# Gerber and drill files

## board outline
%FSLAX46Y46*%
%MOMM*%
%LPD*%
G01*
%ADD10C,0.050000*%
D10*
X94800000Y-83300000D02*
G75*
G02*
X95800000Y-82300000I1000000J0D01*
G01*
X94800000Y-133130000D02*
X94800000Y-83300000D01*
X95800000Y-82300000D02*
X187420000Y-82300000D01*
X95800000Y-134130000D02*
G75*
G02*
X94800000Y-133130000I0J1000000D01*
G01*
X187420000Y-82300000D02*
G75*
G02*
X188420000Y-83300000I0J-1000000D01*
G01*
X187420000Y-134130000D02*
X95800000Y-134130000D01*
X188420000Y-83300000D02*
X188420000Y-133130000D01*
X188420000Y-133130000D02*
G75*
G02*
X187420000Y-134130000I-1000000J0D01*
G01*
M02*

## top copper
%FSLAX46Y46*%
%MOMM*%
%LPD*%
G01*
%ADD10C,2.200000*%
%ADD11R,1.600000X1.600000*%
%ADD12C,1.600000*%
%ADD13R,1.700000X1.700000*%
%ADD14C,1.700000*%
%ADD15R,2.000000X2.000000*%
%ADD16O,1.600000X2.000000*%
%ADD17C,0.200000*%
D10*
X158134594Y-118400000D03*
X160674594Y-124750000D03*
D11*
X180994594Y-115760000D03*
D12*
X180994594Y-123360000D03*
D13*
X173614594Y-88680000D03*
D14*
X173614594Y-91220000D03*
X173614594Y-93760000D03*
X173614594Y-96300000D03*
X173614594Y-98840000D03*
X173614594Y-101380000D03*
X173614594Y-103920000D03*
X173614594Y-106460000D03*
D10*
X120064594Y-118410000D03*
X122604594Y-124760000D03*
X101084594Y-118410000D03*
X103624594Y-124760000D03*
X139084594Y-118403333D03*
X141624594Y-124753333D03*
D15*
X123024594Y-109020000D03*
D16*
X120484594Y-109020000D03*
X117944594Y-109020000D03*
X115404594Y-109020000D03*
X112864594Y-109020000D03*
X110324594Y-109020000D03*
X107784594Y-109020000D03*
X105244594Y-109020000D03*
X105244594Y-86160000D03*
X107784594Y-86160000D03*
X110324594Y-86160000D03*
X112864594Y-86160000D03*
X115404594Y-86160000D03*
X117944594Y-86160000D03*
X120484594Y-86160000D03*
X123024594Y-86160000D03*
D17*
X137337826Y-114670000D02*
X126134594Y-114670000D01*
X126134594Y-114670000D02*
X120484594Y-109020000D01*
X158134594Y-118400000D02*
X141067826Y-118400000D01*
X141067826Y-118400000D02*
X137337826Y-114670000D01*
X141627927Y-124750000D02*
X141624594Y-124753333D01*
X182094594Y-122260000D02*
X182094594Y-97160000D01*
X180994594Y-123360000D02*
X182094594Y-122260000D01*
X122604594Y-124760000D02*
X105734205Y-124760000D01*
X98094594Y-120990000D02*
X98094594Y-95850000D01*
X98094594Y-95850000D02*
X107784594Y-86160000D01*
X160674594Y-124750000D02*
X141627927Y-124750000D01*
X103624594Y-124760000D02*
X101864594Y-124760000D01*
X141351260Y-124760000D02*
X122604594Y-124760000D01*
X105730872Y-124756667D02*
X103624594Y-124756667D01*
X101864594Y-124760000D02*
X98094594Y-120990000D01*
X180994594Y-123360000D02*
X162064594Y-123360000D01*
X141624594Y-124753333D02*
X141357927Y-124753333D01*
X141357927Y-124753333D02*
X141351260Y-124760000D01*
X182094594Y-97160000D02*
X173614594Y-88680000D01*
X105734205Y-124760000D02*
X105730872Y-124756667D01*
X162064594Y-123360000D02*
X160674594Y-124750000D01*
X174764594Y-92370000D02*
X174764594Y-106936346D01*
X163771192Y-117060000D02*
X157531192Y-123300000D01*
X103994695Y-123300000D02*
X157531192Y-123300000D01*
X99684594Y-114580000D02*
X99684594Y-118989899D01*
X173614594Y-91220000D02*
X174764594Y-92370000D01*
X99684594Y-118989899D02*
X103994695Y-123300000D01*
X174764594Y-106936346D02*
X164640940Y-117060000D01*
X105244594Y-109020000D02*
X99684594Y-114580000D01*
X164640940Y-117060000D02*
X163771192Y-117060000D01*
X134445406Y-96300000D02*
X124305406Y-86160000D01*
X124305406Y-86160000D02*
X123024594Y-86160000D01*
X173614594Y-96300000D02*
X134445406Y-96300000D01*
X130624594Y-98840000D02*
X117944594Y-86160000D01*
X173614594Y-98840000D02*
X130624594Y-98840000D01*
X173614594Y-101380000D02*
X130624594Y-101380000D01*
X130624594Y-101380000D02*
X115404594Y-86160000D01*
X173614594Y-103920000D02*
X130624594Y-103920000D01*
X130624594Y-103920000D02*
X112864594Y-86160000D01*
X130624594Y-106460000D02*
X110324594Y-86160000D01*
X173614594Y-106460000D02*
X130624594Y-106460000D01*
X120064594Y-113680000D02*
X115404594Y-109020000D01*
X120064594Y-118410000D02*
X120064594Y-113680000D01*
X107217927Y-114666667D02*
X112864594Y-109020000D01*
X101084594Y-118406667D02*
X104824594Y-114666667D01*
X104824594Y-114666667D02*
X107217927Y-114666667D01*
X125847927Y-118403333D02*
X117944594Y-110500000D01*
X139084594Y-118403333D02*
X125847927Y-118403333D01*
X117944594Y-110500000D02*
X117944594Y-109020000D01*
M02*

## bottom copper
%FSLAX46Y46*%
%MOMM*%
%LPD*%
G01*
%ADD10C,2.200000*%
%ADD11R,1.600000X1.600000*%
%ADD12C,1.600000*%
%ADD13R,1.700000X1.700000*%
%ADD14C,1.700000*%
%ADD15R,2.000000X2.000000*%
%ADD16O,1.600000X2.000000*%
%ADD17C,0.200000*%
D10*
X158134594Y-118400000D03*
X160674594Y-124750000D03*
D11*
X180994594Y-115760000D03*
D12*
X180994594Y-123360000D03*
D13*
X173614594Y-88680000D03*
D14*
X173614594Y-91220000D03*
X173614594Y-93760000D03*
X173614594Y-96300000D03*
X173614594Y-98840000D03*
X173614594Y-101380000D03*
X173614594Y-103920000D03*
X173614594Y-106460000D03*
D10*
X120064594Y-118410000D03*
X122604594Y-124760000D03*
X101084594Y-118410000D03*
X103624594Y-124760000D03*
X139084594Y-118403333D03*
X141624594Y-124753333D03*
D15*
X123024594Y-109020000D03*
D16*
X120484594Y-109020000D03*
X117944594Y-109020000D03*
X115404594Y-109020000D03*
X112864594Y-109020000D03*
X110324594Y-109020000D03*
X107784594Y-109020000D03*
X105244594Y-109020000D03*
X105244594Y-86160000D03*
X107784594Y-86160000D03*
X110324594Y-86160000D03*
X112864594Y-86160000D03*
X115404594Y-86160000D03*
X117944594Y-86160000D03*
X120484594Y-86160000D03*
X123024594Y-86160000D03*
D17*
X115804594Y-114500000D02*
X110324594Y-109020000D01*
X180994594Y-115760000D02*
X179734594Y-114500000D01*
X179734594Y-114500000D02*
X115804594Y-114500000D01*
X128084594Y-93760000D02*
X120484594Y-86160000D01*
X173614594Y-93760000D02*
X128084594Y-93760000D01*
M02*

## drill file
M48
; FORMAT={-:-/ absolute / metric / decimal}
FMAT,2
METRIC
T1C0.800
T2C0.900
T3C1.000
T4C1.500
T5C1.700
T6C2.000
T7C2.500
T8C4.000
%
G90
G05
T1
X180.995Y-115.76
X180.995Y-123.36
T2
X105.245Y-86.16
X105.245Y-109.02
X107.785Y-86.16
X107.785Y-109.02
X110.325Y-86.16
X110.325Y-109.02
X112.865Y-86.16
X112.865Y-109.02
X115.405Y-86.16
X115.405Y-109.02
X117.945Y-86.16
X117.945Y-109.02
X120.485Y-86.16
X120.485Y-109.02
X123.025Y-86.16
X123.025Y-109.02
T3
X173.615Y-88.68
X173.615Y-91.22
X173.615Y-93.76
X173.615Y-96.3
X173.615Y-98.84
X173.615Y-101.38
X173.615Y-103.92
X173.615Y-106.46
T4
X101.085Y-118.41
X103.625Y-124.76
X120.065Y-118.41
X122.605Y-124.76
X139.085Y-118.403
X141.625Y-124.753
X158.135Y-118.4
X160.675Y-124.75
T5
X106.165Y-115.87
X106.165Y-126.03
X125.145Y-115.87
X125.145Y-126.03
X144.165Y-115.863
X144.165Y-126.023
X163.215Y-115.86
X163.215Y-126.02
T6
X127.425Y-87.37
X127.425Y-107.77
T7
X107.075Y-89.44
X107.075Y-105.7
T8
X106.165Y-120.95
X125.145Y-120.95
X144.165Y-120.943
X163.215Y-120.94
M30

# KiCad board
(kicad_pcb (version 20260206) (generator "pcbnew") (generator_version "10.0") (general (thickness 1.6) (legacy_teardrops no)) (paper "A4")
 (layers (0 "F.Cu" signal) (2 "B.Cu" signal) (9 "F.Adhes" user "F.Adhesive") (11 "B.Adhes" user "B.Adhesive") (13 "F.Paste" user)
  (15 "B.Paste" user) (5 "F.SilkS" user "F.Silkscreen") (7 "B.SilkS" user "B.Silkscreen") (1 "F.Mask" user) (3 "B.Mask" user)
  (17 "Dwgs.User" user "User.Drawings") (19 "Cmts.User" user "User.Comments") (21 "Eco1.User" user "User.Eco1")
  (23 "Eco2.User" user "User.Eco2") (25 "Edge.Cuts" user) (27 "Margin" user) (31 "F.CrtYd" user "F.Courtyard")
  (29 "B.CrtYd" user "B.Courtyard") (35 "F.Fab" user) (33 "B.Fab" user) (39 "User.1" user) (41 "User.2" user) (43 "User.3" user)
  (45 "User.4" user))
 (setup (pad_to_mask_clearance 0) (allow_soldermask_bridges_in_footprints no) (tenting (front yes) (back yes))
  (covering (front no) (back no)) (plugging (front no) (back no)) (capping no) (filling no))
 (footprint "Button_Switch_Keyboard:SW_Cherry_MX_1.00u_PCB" (layer "F.Cu") (at 158.134594 118.4 90)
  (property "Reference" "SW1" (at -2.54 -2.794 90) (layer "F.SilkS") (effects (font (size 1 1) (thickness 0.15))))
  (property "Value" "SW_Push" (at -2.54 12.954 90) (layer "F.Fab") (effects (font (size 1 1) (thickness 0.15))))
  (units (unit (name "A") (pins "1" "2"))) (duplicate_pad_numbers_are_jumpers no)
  (pad "" np_thru_hole circle (at -7.62 5.08 90) (size 1.7 1.7) (drill 1.7) (layers "*.Cu" "*.Mask"))
  (pad "" np_thru_hole circle (at -2.54 5.08 90) (size 4 4) (drill 4) (layers "*.Cu" "*.Mask"))
  (pad "" np_thru_hole circle (at 2.54 5.08 90) (size 1.7 1.7) (drill 1.7) (layers "*.Cu" "*.Mask"))
  (pad "1" thru_hole circle (at 0 0 90) (size 2.2 2.2) (drill 1.5) (layers "*.Cu" "*.Mask") (remove_unused_layers no) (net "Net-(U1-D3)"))
  (pad "2" thru_hole circle (at -6.35 2.54 90) (size 2.2 2.2) (drill 1.5) (layers "*.Cu" "*.Mask") (remove_unused_layers no) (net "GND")))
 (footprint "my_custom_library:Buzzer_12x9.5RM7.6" (layer "F.Cu") (at 180.994594 119.56 -90)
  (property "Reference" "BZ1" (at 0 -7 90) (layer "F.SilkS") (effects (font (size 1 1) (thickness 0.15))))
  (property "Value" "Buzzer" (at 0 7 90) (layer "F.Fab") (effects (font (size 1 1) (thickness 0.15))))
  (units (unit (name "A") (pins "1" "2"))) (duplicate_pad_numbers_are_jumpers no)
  (pad "1" thru_hole rect (at -3.8 0 270) (size 1.6 1.6) (drill 0.8) (layers "*.Cu" "*.Mask") (remove_unused_layers no) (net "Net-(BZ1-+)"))
  (pad "2" thru_hole circle (at 3.8 0 270) (size 1.6 1.6) (drill 0.8) (layers "*.Cu" "*.Mask") (remove_unused_layers no) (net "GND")))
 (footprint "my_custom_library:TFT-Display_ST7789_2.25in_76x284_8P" (layer "F.Cu") (at 173.614594 88.68 -90)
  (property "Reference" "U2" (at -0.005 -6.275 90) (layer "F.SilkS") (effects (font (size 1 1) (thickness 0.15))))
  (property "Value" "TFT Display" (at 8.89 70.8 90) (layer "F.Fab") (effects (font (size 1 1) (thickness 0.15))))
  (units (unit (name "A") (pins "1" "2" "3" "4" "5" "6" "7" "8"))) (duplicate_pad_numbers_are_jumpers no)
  (pad "" np_thru_hole circle (at 0.76 66.54 270) (size 2.5 2.5) (drill 2.5) (layers "*.Cu" "*.Mask"))
  (pad "" np_thru_hole circle (at 17.02 66.54 270) (size 2.5 2.5) (drill 2.5) (layers "*.Cu" "*.Mask"))
  (pad "1" thru_hole rect (at 0 0 270) (size 1.7 1.7) (drill 1) (layers "*.Cu" "*.Mask") (remove_unused_layers no) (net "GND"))
  (pad "2" thru_hole circle (at 2.54 0 270) (size 1.7 1.7) (drill 1) (layers "*.Cu" "*.Mask") (remove_unused_layers no) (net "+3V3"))
  (pad "3" thru_hole circle (at 5.08 0 270) (size 1.7 1.7) (drill 1) (layers "*.Cu" "*.Mask") (remove_unused_layers no) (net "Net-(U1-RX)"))
  (pad "4" thru_hole circle (at 7.62 0 270) (size 1.7 1.7) (drill 1) (layers "*.Cu" "*.Mask") (remove_unused_layers no) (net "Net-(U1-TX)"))
  (pad "5" thru_hole circle (at 10.16 0 270) (size 1.7 1.7) (drill 1) (layers "*.Cu" "*.Mask") (remove_unused_layers no)
   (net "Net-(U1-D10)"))
  (pad "6" thru_hole circle (at 12.7 0 270) (size 1.7 1.7) (drill 1) (layers "*.Cu" "*.Mask") (remove_unused_layers no) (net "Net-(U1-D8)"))
  (pad "7" thru_hole circle (at 15.24 0 270) (size 1.7 1.7) (drill 1) (layers "*.Cu" "*.Mask") (remove_unused_layers no) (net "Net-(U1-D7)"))
  (pad "8" thru_hole circle (at 17.78 0 270) (size 1.7 1.7) (drill 1) (layers "*.Cu" "*.Mask") (remove_unused_layers no) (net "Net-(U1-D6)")))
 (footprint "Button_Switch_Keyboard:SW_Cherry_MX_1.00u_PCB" (layer "F.Cu") (at 120.064594 118.41 90)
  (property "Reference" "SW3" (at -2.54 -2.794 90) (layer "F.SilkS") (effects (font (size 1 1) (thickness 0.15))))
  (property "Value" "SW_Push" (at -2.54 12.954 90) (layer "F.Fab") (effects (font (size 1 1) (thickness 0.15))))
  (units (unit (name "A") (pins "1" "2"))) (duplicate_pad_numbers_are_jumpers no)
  (pad "" np_thru_hole circle (at -7.62 5.08 90) (size 1.7 1.7) (drill 1.7) (layers "*.Cu" "*.Mask"))
  (pad "" np_thru_hole circle (at -2.54 5.08 90) (size 4 4) (drill 4) (layers "*.Cu" "*.Mask"))
  (pad "" np_thru_hole circle (at 2.54 5.08 90) (size 1.7 1.7) (drill 1.7) (layers "*.Cu" "*.Mask"))
  (pad "1" thru_hole circle (at 0 0 90) (size 2.2 2.2) (drill 1.5) (layers "*.Cu" "*.Mask") (remove_unused_layers no) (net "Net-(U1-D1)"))
  (pad "2" thru_hole circle (at -6.35 2.54 90) (size 2.2 2.2) (drill 1.5) (layers "*.Cu" "*.Mask") (remove_unused_layers no) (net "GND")))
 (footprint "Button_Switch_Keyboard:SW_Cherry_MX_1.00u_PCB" (layer "F.Cu") (at 101.084594 118.41 90)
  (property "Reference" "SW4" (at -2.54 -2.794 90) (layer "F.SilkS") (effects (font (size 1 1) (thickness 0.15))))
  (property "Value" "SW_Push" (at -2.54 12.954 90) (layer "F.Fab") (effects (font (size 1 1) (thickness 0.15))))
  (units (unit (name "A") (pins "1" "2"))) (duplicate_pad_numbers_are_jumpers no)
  (pad "" np_thru_hole circle (at -7.62 5.08 90) (size 1.7 1.7) (drill 1.7) (layers "*.Cu" "*.Mask"))
  (pad "" np_thru_hole circle (at -2.54 5.08 90) (size 4 4) (drill 4) (layers "*.Cu" "*.Mask"))
  (pad "" np_thru_hole circle (at 2.54 5.08 90) (size 1.7 1.7) (drill 1.7) (layers "*.Cu" "*.Mask"))
  (pad "1" thru_hole circle (at 0 0 90) (size 2.2 2.2) (drill 1.5) (layers "*.Cu" "*.Mask") (remove_unused_layers no) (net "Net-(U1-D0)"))
  (pad "2" thru_hole circle (at -6.35 2.54 90) (size 2.2 2.2) (drill 1.5) (layers "*.Cu" "*.Mask") (remove_unused_layers no) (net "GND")))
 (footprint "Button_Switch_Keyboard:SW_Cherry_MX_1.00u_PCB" (layer "F.Cu") (at 139.084594 118.403333 90)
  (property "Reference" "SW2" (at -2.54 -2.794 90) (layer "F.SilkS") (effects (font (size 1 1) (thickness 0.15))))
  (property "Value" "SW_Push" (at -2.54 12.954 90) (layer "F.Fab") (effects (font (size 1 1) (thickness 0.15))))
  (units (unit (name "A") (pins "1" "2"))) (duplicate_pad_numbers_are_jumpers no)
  (pad "" np_thru_hole circle (at -7.62 5.08 90) (size 1.7 1.7) (drill 1.7) (layers "*.Cu" "*.Mask"))
  (pad "" np_thru_hole circle (at -2.54 5.08 90) (size 4 4) (drill 4) (layers "*.Cu" "*.Mask"))
  (pad "" np_thru_hole circle (at 2.54 5.08 90) (size 1.7 1.7) (drill 1.7) (layers "*.Cu" "*.Mask"))
  (pad "1" thru_hole circle (at 0 0 90) (size 2.2 2.2) (drill 1.5) (layers "*.Cu" "*.Mask") (remove_unused_layers no) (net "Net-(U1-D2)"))
  (pad "2" thru_hole circle (at -6.35 2.54 90) (size 2.2 2.2) (drill 1.5) (layers "*.Cu" "*.Mask") (remove_unused_layers no) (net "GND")))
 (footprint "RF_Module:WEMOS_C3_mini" (layer "B.Cu") (at 123.024594 109.02 90)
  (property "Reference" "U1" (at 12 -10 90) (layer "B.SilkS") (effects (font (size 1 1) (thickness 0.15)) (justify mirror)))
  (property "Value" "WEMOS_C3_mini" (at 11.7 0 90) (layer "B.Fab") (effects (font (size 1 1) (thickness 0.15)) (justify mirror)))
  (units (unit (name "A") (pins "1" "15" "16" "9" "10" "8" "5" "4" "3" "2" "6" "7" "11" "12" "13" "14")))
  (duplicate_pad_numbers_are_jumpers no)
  (pad "" np_thru_hole circle (at 1.25 4.4 90) (size 3 3) (drill 2) (layers "*.Mask"))
  (pad "" np_thru_hole circle (at 21.65 4.4 90) (size 3 3) (drill 2) (layers "*.Mask"))
  (pad "1" thru_hole rect (at 0 0 90) (size 2 2) (drill 0.9) (layers "*.Cu" "*.Mask") (remove_unused_layers no)
   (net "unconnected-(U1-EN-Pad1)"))
  (pad "2" thru_hole oval (at 0 -2.54 90) (size 2 1.6) (drill 0.9) (layers "*.Cu" "*.Mask") (remove_unused_layers no) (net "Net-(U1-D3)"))
  (pad "3" thru_hole oval (at 0 -5.08 90) (size 2 1.6) (drill 0.9) (layers "*.Cu" "*.Mask") (remove_unused_layers no) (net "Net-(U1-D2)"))
  (pad "4" thru_hole oval (at 0 -7.62 90) (size 2 1.6) (drill 0.9) (layers "*.Cu" "*.Mask") (remove_unused_layers no) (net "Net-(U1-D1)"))
  (pad "5" thru_hole oval (at 0 -10.16 90) (size 2 1.6) (drill 0.9) (layers "*.Cu" "*.Mask") (remove_unused_layers no) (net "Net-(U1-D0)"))
  (pad "6" thru_hole oval (at 0 -12.7 90) (size 2 1.6) (drill 0.9) (layers "*.Cu" "*.Mask") (remove_unused_layers no) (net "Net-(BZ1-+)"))
  (pad "7" thru_hole oval (at 0 -15.24 90) (size 2 1.6) (drill 0.9) (layers "*.Cu" "*.Mask") (remove_unused_layers no)
   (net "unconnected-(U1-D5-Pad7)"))
  (pad "8" thru_hole oval (at 0 -17.78 90) (size 2 1.6) (drill 0.9) (layers "*.Cu" "*.Mask") (remove_unused_layers no) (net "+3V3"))
  (pad "9" thru_hole oval (at 22.86 -17.78 90) (size 2 1.6) (drill 0.9) (layers "*.Cu" "*.Mask") (remove_unused_layers no)
   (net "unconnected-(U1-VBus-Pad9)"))
  (pad "10" thru_hole oval (at 22.86 -15.24 90) (size 2 1.6) (drill 0.9) (layers "*.Cu" "*.Mask") (remove_unused_layers no) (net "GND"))
  (pad "11" thru_hole oval (at 22.86 -12.7 90) (size 2 1.6) (drill 0.9) (layers "*.Cu" "*.Mask") (remove_unused_layers no)
   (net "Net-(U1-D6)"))
  (pad "12" thru_hole oval (at 22.86 -10.16 90) (size 2 1.6) (drill 0.9) (layers "*.Cu" "*.Mask") (remove_unused_layers no)
   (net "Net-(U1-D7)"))
  (pad "13" thru_hole oval (at 22.86 -7.62 90) (size 2 1.6) (drill 0.9) (layers "*.Cu" "*.Mask") (remove_unused_layers no)
   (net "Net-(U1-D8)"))
  (pad "14" thru_hole oval (at 22.86 -5.08 90) (size 2 1.6) (drill 0.9) (layers "*.Cu" "*.Mask") (remove_unused_layers no)
   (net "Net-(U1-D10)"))
  (pad "15" thru_hole oval (at 22.86 -2.54 90) (size 2 1.6) (drill 0.9) (layers "*.Cu" "*.Mask") (remove_unused_layers no)
   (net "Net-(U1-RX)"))
  (pad "16" thru_hole oval (at 22.86 0 90) (size 2 1.6) (drill 0.9) (layers "*.Cu" "*.Mask") (remove_unused_layers no) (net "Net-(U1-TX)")))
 (gr_arc (start 94.8 83.3) (mid 95.092893 82.592893) (end 95.8 82.3) (stroke (width 0.05) (type default)) (layer "Edge.Cuts"))
 (gr_line (start 94.8 133.13) (end 94.8 83.3) (stroke (width 0.05) (type default)) (layer "Edge.Cuts"))
 (gr_line (start 95.8 82.3) (end 187.42 82.3) (stroke (width 0.05) (type default)) (layer "Edge.Cuts"))
 (gr_arc (start 95.8 134.13) (mid 95.092893 133.837107) (end 94.8 133.13) (stroke (width 0.05) (type default)) (layer "Edge.Cuts"))
 (gr_arc (start 187.42 82.3) (mid 188.127107 82.592893) (end 188.42 83.3) (stroke (width 0.05) (type default)) (layer "Edge.Cuts"))
 (gr_line (start 187.42 134.13) (end 95.8 134.13) (stroke (width 0.05) (type default)) (layer "Edge.Cuts"))
 (gr_line (start 188.42 83.3) (end 188.42 133.13) (stroke (width 0.05) (type default)) (layer "Edge.Cuts"))
 (gr_arc (start 188.42 133.13) (mid 188.127107 133.837107) (end 187.42 134.13) (stroke (width 0.05) (type default)) (layer "Edge.Cuts"))
 (segment (start 137.337826 114.67) (end 126.134594 114.67) (width 0.2) (layer "F.Cu") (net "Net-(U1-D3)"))
 (segment (start 126.134594 114.67) (end 120.484594 109.02) (width 0.2) (layer "F.Cu") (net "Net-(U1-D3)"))
 (segment (start 158.134594 118.4) (end 141.067826 118.4) (width 0.2) (layer "F.Cu") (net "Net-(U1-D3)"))
 (segment (start 141.067826 118.4) (end 137.337826 114.67) (width 0.2) (layer "F.Cu") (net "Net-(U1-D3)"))
 (segment (start 141.627927 124.75) (end 141.624594 124.753333) (width 0.2) (layer "F.Cu") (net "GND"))
 (segment (start 182.094594 122.26) (end 182.094594 97.16) (width 0.2) (layer "F.Cu") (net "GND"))
 (segment (start 180.994594 123.36) (end 182.094594 122.26) (width 0.2) (layer "F.Cu") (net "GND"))
 (segment (start 122.604594 124.76) (end 105.734205 124.76) (width 0.2) (layer "F.Cu") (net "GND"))
 (segment (start 98.094594 120.99) (end 98.094594 95.85) (width 0.2) (layer "F.Cu") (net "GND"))
 (segment (start 98.094594 95.85) (end 107.784594 86.16) (width 0.2) (layer "F.Cu") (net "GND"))
 (segment (start 160.674594 124.75) (end 141.627927 124.75) (width 0.2) (layer "F.Cu") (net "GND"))
 (segment (start 103.624594 124.76) (end 101.864594 124.76) (width 0.2) (layer "F.Cu") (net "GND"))
 (segment (start 141.35126 124.76) (end 122.604594 124.76) (width 0.2) (layer "F.Cu") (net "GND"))
 (segment (start 105.730872 124.756667) (end 103.624594 124.756667) (width 0.2) (layer "F.Cu") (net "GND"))
 (segment (start 101.864594 124.76) (end 98.094594 120.99) (width 0.2) (layer "F.Cu") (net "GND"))
 (segment (start 180.994594 123.36) (end 162.064594 123.36) (width 0.2) (layer "F.Cu") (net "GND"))
 (segment (start 141.624594 124.753333) (end 141.357927 124.753333) (width 0.2) (layer "F.Cu") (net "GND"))
 (segment (start 141.357927 124.753333) (end 141.35126 124.76) (width 0.2) (layer "F.Cu") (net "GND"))
 (segment (start 182.094594 97.16) (end 173.614594 88.68) (width 0.2) (layer "F.Cu") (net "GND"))
 (segment (start 105.734205 124.76) (end 105.730872 124.756667) (width 0.2) (layer "F.Cu") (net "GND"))
 (segment (start 162.064594 123.36) (end 160.674594 124.75) (width 0.2) (layer "F.Cu") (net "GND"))
 (segment (start 115.804594 114.5) (end 110.324594 109.02) (width 0.2) (layer "B.Cu") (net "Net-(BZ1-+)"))
 (segment (start 180.994594 115.76) (end 179.734594 114.5) (width 0.2) (layer "B.Cu") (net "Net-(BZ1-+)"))
 (segment (start 179.734594 114.5) (end 115.804594 114.5) (width 0.2) (layer "B.Cu") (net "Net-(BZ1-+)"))
 (segment (start 174.764594 92.37) (end 174.764594 106.936346) (width 0.2) (layer "F.Cu") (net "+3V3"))
 (segment (start 163.771192 117.06) (end 157.531192 123.3) (width 0.2) (layer "F.Cu") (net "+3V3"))
 (segment (start 103.994695 123.3) (end 157.531192 123.3) (width 0.2) (layer "F.Cu") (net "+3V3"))
 (segment (start 99.684594 114.58) (end 99.684594 118.989899) (width 0.2) (layer "F.Cu") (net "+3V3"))
 (segment (start 173.614594 91.22) (end 174.764594 92.37) (width 0.2) (layer "F.Cu") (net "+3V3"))
 (segment (start 99.684594 118.989899) (end 103.994695 123.3) (width 0.2) (layer "F.Cu") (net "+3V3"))
 (segment (start 174.764594 106.936346) (end 164.64094 117.06) (width 0.2) (layer "F.Cu") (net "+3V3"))
 (segment (start 105.244594 109.02) (end 99.684594 114.58) (width 0.2) (layer "F.Cu") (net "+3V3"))
 (segment (start 164.64094 117.06) (end 163.771192 117.06) (width 0.2) (layer "F.Cu") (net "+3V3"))
 (segment (start 128.084594 93.76) (end 120.484594 86.16) (width 0.2) (layer "B.Cu") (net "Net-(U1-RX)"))
 (segment (start 173.614594 93.76) (end 128.084594 93.76) (width 0.2) (layer "B.Cu") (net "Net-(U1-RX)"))
 (segment (start 134.445406 96.3) (end 124.305406 86.16) (width 0.2) (layer "F.Cu") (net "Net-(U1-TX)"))
 (segment (start 124.305406 86.16) (end 123.024594 86.16) (width 0.2) (layer "F.Cu") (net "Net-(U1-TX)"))
 (segment (start 173.614594 96.3) (end 134.445406 96.3) (width 0.2) (layer "F.Cu") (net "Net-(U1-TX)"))
 (segment (start 130.624594 98.84) (end 117.944594 86.16) (width 0.2) (layer "F.Cu") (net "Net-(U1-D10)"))
 (segment (start 173.614594 98.84) (end 130.624594 98.84) (width 0.2) (layer "F.Cu") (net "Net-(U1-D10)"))
 (segment (start 173.614594 101.38) (end 130.624594 101.38) (width 0.2) (layer "F.Cu") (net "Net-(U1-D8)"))
 (segment (start 130.624594 101.38) (end 115.404594 86.16) (width 0.2) (layer "F.Cu") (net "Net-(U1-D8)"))
 (segment (start 173.614594 103.92) (end 130.624594 103.92) (width 0.2) (layer "F.Cu") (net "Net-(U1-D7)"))
 (segment (start 130.624594 103.92) (end 112.864594 86.16) (width 0.2) (layer "F.Cu") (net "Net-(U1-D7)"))
 (segment (start 130.624594 106.46) (end 110.324594 86.16) (width 0.2) (layer "F.Cu") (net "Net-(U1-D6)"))
 (segment (start 173.614594 106.46) (end 130.624594 106.46) (width 0.2) (layer "F.Cu") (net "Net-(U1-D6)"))
 (segment (start 120.064594 113.68) (end 115.404594 109.02) (width 0.2) (layer "F.Cu") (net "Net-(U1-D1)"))
 (segment (start 120.064594 118.41) (end 120.064594 113.68) (width 0.2) (layer "F.Cu") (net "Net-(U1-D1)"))
 (segment (start 107.217927 114.666667) (end 112.864594 109.02) (width 0.2) (layer "F.Cu") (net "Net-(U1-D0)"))
 (segment (start 101.084594 118.406667) (end 104.824594 114.666667) (width 0.2) (layer "F.Cu") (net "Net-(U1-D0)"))
 (segment (start 104.824594 114.666667) (end 107.217927 114.666667) (width 0.2) (layer "F.Cu") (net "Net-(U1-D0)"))
 (segment (start 125.847927 118.403333) (end 117.944594 110.5) (width 0.2) (layer "F.Cu") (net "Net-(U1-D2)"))
 (segment (start 139.084594 118.403333) (end 125.847927 118.403333) (width 0.2) (layer "F.Cu") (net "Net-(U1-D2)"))
 (segment (start 117.944594 110.5) (end 117.944594 109.02) (width 0.2) (layer "F.Cu") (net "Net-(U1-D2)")))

